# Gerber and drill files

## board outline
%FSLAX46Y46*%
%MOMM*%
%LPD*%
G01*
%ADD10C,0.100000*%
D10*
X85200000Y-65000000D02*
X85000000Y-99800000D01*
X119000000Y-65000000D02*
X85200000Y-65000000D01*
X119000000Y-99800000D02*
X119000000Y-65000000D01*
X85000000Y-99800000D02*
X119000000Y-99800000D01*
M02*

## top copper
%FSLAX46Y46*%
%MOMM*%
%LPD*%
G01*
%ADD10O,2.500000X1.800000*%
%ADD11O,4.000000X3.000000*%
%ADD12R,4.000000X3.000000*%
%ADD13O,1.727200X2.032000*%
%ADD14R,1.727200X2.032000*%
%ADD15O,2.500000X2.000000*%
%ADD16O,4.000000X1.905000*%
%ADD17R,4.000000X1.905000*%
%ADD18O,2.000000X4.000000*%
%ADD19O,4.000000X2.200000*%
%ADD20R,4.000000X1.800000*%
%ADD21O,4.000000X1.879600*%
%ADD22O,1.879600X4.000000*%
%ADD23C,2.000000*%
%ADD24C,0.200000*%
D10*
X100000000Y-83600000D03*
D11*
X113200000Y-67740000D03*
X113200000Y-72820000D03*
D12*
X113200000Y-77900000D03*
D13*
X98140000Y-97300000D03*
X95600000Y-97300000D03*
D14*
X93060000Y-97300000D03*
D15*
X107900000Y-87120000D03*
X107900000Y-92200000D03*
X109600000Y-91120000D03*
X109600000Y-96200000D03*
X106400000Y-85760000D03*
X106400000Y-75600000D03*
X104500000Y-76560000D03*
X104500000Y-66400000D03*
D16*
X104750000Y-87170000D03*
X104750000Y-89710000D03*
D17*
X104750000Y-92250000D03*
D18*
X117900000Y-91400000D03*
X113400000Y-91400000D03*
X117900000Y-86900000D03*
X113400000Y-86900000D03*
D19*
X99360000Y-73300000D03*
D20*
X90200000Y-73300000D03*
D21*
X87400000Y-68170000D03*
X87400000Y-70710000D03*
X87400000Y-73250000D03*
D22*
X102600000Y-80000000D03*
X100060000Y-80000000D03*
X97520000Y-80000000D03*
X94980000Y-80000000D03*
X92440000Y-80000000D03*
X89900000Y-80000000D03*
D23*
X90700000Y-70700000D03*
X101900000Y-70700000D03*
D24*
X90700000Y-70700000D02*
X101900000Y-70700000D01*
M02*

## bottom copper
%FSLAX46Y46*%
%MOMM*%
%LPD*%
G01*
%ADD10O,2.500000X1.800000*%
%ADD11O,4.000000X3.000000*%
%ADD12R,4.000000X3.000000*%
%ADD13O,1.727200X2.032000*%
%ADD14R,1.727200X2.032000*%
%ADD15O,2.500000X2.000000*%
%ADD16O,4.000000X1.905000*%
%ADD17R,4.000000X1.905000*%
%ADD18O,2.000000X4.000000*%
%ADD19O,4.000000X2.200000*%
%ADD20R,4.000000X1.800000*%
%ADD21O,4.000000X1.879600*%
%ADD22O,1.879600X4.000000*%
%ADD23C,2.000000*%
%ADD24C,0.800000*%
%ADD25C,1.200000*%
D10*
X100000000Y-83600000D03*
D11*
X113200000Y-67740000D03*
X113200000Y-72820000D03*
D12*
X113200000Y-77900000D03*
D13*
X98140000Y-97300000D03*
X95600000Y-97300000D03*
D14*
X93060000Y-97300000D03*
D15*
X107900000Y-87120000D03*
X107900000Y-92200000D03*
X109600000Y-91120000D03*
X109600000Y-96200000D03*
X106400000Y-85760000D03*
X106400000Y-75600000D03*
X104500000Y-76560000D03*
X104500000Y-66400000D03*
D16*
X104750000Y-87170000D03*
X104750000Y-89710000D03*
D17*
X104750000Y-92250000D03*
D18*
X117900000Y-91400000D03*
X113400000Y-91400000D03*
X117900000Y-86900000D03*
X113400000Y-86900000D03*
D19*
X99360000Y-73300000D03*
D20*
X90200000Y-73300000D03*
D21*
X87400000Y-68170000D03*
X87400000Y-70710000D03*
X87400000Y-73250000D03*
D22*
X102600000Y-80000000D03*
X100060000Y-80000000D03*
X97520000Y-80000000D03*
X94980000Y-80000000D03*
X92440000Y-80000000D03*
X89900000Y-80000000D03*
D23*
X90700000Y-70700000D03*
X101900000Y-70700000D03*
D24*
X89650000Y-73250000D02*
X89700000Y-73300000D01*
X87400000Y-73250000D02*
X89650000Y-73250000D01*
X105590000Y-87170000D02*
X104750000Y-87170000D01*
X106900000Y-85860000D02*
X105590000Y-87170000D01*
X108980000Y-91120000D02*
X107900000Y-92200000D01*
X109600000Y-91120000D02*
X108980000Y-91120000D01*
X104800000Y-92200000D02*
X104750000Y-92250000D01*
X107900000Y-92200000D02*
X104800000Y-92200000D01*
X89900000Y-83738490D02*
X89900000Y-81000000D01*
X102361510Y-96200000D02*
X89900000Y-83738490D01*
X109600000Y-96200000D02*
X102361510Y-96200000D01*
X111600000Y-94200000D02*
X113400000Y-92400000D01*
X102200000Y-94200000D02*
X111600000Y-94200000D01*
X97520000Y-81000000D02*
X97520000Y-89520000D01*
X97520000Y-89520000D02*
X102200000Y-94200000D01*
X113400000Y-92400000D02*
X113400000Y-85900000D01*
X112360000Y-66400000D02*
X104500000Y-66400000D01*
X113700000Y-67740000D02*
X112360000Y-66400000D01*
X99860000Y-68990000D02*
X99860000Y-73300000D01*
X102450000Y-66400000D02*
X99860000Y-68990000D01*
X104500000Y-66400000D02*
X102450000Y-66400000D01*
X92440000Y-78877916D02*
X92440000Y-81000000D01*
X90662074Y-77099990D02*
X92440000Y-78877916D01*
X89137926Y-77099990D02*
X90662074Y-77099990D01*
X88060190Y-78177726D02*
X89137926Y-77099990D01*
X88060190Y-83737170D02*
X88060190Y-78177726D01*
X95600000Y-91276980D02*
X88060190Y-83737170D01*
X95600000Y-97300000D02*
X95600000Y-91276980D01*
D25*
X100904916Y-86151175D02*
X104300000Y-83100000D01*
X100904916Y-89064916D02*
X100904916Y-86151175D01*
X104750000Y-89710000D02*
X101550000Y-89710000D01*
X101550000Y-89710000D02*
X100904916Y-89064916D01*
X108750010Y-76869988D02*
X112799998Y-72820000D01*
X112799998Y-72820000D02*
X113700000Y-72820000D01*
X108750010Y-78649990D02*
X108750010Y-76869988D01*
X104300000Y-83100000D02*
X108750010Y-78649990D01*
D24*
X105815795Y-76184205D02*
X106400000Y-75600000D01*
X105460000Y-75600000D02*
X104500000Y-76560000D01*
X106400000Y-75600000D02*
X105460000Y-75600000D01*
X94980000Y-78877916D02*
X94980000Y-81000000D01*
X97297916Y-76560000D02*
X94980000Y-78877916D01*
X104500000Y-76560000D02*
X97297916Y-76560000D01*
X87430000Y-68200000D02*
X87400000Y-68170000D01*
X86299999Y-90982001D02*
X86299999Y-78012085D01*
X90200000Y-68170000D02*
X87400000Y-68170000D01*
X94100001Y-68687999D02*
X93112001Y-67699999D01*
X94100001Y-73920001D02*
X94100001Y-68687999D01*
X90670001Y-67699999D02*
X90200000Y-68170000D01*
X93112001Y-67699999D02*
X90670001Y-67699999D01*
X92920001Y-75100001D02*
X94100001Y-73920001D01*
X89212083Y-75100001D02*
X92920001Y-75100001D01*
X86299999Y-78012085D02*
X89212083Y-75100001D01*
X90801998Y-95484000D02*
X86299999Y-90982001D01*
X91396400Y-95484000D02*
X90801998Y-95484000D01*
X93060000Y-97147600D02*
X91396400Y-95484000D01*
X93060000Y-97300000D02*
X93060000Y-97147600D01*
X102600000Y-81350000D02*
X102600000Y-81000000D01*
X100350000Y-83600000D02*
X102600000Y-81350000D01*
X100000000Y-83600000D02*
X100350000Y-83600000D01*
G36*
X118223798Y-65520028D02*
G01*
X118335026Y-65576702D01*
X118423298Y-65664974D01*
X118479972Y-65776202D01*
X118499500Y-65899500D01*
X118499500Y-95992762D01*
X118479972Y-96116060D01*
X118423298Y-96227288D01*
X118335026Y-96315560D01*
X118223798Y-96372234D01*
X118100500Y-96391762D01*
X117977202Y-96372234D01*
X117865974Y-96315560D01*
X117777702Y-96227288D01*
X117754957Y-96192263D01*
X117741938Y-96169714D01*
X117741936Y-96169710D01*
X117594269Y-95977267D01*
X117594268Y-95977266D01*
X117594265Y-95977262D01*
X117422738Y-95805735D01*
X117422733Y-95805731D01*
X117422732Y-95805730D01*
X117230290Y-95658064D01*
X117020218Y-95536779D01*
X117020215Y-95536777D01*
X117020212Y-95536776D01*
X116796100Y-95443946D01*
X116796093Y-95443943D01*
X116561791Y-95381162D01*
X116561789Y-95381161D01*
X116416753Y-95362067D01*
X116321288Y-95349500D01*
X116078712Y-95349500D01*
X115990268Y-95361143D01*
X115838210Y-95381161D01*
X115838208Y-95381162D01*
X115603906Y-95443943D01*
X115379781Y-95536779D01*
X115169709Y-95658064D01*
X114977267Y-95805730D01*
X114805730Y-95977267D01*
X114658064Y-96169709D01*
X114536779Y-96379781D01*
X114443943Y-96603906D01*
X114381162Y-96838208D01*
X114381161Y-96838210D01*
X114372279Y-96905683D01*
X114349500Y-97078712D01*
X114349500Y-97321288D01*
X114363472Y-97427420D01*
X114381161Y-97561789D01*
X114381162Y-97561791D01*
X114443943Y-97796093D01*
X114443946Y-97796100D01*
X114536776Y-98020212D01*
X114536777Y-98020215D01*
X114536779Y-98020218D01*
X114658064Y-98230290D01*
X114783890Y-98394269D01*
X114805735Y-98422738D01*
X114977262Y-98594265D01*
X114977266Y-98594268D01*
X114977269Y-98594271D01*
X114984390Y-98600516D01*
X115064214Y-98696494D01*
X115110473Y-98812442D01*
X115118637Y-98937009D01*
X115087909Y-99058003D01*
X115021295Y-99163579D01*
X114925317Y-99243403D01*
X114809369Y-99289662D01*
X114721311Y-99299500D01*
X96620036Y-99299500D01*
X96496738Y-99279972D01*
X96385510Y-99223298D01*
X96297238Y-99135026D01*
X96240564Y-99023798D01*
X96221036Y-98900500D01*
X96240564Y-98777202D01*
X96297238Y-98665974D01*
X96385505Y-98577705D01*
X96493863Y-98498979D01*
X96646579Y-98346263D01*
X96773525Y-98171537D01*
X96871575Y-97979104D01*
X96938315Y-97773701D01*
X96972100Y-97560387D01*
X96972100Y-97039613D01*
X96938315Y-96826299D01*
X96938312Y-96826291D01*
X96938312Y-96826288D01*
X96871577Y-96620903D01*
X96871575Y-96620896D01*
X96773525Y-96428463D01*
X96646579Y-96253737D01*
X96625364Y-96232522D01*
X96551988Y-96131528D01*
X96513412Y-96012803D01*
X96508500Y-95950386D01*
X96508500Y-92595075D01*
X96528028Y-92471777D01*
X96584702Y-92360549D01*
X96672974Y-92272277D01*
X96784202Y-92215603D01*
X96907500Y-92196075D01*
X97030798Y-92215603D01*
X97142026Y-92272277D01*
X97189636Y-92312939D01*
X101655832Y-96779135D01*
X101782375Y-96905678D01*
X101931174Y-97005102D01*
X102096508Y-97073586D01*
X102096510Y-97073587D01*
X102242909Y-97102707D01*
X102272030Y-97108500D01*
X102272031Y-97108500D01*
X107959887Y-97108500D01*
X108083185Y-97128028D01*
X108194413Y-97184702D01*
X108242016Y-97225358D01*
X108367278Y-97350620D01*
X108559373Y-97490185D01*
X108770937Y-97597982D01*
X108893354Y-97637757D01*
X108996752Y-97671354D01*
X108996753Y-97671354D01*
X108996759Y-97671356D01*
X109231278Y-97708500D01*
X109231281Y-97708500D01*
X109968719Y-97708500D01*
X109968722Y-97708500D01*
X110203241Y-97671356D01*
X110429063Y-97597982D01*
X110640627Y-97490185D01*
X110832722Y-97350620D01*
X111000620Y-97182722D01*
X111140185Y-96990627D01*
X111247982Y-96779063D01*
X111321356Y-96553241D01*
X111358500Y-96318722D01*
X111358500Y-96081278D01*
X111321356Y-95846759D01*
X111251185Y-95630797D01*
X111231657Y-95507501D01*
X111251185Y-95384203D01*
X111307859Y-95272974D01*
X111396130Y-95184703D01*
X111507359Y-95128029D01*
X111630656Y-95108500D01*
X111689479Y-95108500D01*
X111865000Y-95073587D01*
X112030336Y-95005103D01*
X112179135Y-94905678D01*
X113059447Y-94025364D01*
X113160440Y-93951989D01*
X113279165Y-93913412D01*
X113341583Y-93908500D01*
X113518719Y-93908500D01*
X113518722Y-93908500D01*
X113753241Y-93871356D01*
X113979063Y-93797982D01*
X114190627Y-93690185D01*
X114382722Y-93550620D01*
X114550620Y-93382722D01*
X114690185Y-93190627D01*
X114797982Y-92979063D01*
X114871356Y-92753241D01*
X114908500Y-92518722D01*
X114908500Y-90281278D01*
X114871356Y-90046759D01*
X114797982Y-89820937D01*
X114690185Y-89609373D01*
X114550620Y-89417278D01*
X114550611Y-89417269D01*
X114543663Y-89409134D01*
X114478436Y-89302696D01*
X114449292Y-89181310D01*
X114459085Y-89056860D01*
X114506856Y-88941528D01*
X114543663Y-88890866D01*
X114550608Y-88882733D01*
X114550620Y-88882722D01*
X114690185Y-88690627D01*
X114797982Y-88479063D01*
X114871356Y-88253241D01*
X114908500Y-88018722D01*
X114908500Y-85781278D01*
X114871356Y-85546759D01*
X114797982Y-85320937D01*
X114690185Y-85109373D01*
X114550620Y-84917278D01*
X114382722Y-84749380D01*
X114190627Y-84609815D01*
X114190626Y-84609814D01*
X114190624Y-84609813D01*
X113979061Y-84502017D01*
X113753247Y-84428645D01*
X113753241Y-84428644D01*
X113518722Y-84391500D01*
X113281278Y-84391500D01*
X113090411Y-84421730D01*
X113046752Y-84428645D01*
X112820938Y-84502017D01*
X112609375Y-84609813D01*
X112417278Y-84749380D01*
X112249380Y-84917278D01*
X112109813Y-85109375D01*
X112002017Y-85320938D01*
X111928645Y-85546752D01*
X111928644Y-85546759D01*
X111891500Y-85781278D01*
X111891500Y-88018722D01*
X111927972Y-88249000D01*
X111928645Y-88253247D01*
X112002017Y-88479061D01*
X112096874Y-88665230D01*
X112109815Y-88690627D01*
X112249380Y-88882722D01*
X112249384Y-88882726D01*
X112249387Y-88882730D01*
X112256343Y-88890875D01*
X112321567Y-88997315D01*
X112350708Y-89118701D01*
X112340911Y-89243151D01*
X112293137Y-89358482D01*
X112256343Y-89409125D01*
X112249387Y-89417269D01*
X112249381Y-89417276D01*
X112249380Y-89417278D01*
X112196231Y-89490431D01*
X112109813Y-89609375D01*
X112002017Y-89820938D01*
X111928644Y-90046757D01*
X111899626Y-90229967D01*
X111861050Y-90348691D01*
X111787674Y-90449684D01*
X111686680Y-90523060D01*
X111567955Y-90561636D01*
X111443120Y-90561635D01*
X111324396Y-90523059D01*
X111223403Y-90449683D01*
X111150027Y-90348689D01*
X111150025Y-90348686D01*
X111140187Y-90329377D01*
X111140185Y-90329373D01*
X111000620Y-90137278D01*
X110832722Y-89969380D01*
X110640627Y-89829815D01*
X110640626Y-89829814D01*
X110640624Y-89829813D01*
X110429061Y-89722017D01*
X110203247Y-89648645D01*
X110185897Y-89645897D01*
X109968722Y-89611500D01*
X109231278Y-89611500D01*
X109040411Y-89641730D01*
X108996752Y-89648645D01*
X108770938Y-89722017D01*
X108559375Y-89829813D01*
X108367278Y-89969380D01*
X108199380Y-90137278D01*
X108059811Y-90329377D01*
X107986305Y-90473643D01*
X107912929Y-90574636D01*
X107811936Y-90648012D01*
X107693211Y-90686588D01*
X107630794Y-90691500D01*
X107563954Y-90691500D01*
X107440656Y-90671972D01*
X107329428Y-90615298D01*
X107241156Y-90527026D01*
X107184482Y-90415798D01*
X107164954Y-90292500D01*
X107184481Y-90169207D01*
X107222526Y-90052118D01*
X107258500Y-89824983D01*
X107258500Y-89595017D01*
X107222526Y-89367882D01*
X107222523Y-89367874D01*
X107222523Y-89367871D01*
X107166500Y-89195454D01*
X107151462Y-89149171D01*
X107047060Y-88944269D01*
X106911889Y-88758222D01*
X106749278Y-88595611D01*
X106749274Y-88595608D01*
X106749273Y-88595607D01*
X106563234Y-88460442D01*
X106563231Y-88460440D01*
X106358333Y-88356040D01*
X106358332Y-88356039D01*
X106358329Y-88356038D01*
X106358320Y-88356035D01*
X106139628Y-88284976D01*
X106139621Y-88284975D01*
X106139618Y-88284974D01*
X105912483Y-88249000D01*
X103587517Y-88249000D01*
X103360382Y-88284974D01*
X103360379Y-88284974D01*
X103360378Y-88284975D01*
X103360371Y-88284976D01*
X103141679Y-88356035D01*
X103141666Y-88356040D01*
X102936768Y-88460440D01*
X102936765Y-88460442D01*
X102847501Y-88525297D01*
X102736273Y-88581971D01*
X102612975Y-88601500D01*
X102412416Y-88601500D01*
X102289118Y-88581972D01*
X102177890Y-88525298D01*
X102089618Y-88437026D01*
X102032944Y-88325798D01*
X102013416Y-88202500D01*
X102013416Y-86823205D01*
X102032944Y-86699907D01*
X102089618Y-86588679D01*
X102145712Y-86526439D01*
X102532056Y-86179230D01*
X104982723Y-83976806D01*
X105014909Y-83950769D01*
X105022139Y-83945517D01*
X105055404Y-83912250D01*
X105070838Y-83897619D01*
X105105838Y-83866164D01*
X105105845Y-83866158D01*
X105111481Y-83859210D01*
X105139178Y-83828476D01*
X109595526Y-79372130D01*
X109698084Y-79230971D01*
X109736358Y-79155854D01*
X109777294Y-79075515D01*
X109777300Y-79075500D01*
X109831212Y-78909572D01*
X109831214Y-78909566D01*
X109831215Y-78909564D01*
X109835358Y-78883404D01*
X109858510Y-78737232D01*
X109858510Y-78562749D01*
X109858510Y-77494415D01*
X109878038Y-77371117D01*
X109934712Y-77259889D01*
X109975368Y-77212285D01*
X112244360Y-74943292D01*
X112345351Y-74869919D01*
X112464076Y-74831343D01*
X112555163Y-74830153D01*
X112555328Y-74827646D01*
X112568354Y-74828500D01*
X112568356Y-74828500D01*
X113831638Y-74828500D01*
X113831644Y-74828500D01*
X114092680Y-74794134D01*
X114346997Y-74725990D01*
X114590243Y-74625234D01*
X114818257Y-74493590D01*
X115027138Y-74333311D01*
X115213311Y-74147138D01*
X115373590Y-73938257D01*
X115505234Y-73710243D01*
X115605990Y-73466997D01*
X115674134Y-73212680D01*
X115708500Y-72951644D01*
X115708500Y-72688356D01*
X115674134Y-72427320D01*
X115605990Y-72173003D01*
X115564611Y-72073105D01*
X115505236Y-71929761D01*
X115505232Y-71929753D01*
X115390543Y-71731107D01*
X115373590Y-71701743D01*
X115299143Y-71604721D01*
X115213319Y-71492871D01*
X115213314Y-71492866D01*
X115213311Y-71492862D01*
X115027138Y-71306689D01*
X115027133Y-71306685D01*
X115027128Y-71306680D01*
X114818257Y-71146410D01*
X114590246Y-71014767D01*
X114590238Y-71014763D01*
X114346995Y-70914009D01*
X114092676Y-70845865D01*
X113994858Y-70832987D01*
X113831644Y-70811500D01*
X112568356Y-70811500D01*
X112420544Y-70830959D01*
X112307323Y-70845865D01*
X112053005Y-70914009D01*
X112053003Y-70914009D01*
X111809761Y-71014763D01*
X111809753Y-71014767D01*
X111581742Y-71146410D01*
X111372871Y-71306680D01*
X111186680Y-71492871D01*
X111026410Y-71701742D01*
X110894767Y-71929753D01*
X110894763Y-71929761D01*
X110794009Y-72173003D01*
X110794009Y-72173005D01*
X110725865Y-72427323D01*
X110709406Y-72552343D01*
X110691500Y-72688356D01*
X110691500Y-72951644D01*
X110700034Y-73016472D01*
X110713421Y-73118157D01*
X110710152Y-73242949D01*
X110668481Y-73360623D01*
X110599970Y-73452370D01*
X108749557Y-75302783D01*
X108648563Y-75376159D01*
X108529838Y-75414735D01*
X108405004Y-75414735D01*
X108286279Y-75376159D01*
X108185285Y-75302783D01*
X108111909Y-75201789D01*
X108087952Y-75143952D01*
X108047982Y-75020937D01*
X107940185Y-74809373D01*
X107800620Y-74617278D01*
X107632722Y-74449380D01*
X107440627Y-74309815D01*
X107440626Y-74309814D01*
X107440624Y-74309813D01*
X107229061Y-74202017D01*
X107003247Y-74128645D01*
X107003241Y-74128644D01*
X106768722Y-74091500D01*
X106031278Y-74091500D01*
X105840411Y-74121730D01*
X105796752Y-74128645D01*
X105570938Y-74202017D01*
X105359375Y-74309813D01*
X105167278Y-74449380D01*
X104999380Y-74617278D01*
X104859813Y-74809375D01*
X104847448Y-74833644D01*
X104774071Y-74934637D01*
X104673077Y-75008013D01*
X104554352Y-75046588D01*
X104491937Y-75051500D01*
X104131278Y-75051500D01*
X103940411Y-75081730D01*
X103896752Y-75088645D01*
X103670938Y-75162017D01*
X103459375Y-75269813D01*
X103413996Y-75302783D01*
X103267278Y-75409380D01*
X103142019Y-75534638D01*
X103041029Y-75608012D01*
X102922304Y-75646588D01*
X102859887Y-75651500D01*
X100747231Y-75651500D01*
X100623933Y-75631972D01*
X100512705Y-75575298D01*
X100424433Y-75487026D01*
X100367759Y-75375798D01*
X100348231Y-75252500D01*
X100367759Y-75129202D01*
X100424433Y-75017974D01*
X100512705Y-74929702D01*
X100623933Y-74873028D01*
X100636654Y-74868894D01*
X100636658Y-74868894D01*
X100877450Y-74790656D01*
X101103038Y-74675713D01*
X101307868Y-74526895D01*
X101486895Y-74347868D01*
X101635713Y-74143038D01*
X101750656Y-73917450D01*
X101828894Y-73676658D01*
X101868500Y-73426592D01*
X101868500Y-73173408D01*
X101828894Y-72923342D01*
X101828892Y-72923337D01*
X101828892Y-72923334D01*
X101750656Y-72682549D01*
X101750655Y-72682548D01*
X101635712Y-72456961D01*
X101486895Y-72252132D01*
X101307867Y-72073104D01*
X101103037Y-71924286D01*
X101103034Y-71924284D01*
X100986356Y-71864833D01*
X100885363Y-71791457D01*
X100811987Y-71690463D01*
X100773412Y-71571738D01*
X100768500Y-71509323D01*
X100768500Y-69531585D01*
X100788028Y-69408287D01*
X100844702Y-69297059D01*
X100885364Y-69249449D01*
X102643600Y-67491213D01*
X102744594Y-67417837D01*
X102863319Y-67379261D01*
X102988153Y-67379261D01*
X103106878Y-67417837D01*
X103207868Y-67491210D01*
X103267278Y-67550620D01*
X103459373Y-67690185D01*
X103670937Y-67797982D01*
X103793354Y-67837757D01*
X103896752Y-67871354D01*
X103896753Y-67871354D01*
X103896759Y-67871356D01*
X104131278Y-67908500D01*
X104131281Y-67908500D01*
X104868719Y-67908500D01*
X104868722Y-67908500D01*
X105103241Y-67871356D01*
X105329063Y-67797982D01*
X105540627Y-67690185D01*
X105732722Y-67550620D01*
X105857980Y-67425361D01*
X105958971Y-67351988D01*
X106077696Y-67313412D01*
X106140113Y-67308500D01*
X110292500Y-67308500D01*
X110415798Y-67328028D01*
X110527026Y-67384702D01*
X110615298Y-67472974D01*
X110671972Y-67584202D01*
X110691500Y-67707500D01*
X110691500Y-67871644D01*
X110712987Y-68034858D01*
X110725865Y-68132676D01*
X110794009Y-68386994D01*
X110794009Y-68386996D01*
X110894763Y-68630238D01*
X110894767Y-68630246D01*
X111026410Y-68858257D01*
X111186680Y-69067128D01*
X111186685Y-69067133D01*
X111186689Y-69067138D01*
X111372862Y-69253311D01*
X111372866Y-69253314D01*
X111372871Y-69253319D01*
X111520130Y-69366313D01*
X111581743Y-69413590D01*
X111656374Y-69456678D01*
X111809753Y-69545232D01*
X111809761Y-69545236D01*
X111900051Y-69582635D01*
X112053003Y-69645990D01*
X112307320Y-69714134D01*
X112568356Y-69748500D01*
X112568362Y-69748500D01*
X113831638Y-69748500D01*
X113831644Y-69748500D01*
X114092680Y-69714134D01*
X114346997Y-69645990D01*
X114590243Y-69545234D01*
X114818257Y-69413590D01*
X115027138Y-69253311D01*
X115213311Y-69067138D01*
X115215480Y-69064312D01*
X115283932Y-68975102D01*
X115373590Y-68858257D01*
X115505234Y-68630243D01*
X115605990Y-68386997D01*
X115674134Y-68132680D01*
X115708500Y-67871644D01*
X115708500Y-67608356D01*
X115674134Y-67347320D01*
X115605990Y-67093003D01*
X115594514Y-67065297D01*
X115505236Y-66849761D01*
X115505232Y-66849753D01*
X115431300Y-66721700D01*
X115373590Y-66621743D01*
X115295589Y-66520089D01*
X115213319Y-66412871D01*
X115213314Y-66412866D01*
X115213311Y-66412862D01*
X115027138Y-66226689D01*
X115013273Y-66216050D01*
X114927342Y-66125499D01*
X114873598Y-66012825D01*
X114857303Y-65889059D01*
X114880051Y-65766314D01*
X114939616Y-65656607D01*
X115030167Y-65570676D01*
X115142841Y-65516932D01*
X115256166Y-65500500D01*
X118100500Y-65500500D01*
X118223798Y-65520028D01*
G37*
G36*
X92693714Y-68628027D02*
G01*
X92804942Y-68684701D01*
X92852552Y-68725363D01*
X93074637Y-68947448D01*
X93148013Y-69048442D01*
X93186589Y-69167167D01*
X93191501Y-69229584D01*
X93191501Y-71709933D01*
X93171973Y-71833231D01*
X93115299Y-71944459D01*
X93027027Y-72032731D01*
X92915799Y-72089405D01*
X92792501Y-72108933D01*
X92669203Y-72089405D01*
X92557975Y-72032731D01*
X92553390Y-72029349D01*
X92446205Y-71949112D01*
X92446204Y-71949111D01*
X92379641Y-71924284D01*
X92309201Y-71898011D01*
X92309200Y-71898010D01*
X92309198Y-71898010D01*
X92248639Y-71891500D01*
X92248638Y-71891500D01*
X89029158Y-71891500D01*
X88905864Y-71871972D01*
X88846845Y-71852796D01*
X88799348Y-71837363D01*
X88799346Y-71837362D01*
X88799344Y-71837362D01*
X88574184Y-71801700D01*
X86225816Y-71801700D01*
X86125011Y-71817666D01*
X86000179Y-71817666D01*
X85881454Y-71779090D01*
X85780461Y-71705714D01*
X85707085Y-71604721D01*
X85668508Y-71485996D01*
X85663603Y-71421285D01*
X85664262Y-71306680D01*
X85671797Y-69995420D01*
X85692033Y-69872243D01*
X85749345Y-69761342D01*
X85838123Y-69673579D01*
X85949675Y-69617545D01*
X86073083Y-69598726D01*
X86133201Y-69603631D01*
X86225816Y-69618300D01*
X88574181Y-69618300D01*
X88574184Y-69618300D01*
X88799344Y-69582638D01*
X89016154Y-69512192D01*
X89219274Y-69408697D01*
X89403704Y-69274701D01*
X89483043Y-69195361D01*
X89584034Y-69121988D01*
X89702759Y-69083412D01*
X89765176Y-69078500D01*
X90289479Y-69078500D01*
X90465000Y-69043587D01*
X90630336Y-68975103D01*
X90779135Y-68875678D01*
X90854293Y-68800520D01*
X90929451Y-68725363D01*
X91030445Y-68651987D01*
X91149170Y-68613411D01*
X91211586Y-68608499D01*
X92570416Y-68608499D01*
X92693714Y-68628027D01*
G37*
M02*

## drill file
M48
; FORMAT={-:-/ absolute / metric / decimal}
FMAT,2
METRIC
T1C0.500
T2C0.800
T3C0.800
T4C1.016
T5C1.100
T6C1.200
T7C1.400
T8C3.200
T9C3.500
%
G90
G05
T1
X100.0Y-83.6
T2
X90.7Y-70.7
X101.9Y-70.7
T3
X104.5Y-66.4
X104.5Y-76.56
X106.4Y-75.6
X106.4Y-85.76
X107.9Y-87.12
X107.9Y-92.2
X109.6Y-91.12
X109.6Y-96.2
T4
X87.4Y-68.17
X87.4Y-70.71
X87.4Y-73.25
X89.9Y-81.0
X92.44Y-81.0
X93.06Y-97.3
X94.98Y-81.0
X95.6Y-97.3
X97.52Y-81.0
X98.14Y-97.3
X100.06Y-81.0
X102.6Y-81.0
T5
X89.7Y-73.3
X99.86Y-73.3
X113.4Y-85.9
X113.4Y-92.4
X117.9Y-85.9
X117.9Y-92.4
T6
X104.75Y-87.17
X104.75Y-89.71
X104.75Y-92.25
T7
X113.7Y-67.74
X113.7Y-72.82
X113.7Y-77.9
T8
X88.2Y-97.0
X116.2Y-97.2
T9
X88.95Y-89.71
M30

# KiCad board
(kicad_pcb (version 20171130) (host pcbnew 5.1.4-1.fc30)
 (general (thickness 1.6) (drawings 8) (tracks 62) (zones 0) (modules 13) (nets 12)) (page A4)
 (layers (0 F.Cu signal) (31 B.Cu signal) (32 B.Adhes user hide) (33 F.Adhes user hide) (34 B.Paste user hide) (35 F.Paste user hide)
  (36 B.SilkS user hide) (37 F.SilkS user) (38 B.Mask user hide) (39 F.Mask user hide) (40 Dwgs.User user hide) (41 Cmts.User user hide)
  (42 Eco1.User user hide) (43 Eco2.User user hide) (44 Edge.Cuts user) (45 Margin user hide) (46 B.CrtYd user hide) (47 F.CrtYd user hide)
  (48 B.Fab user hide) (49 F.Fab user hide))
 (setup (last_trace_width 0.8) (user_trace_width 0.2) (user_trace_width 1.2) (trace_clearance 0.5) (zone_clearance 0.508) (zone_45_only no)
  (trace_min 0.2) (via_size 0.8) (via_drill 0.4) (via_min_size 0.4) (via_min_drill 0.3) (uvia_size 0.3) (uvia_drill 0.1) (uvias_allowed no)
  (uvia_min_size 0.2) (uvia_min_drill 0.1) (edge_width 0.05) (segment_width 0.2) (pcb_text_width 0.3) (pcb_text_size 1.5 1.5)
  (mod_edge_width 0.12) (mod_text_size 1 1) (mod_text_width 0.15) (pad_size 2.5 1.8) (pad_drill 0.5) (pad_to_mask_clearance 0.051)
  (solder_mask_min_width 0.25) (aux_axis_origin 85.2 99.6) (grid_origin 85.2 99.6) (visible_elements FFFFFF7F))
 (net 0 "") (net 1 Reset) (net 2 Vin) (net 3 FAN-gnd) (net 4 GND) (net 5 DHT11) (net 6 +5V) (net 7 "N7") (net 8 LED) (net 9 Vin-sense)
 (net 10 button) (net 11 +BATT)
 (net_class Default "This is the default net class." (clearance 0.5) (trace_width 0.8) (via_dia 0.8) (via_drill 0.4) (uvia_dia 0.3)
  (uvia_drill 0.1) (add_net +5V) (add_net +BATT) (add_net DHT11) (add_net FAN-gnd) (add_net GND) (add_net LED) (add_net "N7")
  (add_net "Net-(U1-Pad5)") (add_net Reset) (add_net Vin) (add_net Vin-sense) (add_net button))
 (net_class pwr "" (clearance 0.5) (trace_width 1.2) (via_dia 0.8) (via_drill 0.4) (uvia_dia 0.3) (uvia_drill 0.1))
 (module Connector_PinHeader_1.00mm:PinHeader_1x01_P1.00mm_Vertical (layer F.Cu) (at 100 83.6)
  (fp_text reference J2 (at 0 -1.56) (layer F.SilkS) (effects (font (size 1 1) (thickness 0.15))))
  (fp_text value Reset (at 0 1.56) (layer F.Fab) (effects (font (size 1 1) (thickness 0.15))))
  (pad 1 thru_hole oval (at 0 0) (size 2.5 1.8) (drill 0.5) (layers *.Cu *.Mask) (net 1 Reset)))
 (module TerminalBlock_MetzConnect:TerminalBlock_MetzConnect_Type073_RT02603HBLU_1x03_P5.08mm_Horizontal (layer F.Cu) (at 113.7 77.9 90)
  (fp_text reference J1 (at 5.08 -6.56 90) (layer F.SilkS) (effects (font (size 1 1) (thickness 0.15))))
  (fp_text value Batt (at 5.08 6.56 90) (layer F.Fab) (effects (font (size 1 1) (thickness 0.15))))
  (pad 3 thru_hole oval (at 10.16 0 90) (size 3 4) (drill 1.4 (offset 0 -0.5)) (layers *.Cu *.Mask) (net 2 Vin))
  (pad 2 thru_hole oval (at 5.08 0 90) (size 3 4) (drill 1.4 (offset 0 -0.5)) (layers *.Cu *.Mask) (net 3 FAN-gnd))
  (pad 1 thru_hole rect (at 0 0 90) (size 3 4) (drill 1.4 (offset 0 -0.5)) (layers *.Cu *.Mask) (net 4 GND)))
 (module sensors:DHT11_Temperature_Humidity (layer F.Cu) (at 95.6 97.3)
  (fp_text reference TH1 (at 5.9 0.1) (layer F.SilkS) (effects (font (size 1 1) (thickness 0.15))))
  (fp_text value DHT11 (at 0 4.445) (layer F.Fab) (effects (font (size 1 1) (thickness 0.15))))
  (pad 3 thru_hole oval (at 2.54 0 90) (size 2.032 1.7272) (drill 1.016) (layers *.Cu *.Mask F.SilkS) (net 4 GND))
  (pad 2 thru_hole oval (at 0 0 90) (size 2.032 1.7272) (drill 1.016) (layers *.Cu *.Mask F.SilkS) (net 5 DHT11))
  (pad 1 thru_hole rect (at -2.54 0 90) (size 2.032 1.7272) (drill 1.016) (layers *.Cu *.Mask F.SilkS) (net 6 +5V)))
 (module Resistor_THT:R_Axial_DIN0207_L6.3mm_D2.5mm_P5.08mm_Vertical (layer F.Cu) (at 107.9 92.2 90)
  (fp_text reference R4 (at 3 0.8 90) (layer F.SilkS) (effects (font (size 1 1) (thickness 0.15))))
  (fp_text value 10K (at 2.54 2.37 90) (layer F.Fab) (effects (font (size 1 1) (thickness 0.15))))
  (pad 2 thru_hole oval (at 5.08 0 90) (size 2 2.5) (drill 0.8) (layers *.Cu *.Mask) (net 4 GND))
  (pad 1 thru_hole oval (at 0 0 90) (size 2 2.5) (drill 0.8) (layers *.Cu *.Mask) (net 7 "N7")))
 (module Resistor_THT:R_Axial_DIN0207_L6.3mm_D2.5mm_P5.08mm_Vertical (layer F.Cu) (at 109.6 96.2 90)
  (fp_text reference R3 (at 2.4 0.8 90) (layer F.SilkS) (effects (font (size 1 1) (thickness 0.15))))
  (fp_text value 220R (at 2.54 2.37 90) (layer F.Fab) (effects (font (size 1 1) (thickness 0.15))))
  (pad 2 thru_hole oval (at 5.08 0 90) (size 2 2.5) (drill 0.8) (layers *.Cu *.Mask) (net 7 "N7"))
  (pad 1 thru_hole oval (at 0 0 90) (size 2 2.5) (drill 0.8) (layers *.Cu *.Mask) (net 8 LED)))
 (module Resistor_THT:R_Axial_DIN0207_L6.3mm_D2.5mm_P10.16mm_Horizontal (layer F.Cu) (at 106.4 75.6 270)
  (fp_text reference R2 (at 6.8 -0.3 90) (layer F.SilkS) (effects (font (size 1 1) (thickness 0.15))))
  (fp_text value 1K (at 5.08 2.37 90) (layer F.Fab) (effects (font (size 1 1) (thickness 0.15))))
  (pad 2 thru_hole oval (at 10.16 0 270) (size 2 2.5) (drill 0.8) (layers *.Cu *.Mask) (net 4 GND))
  (pad 1 thru_hole oval (at 0 0 270) (size 2 2.5) (drill 0.8) (layers *.Cu *.Mask) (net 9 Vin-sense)))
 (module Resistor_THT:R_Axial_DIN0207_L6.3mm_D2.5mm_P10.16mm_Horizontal (layer F.Cu) (at 104.5 66.4 270)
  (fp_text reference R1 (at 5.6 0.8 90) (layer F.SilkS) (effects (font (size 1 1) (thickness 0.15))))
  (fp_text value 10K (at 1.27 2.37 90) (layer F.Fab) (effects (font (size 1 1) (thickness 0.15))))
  (pad 2 thru_hole oval (at 10.16 0 270) (size 2 2.5) (drill 0.8) (layers *.Cu *.Mask) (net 9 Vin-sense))
  (pad 1 thru_hole oval (at 0 0 270) (size 2 2.5) (drill 0.8) (layers *.Cu *.Mask) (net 2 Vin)))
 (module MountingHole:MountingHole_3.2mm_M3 (layer F.Cu) (at 116.2 97.2)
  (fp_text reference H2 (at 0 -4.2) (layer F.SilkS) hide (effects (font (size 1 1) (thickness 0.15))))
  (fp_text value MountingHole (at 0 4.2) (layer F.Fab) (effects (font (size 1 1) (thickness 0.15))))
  (pad 1 np_thru_hole circle (at 0 0) (size 3.2 3.2) (drill 3.2) (layers *.Cu *.Mask)))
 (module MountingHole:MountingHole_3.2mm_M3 (layer F.Cu) (at 88.2 97)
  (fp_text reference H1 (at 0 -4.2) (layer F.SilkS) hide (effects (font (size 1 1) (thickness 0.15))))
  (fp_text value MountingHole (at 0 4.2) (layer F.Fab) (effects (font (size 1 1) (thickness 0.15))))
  (pad 1 np_thru_hole circle (at 0 0) (size 3.2 3.2) (drill 3.2) (layers *.Cu *.Mask)))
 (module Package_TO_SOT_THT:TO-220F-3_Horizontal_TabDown (layer F.Cu) (at 104.75 92.25 90)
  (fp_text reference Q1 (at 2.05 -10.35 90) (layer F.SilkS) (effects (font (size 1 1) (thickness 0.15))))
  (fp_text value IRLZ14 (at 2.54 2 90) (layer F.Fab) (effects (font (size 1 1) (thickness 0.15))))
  (pad 3 thru_hole oval (at 5.08 0 90) (size 1.905 4) (drill 1.2) (layers *.Cu *.Mask) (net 4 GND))
  (pad 2 thru_hole oval (at 2.54 0 90) (size 1.905 4) (drill 1.2) (layers *.Cu *.Mask) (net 3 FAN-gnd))
  (pad 1 thru_hole rect (at 0 0 90) (size 1.905 4) (drill 1.2) (layers *.Cu *.Mask) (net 7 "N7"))
  (pad "" np_thru_hole oval (at 2.54 -15.8 90) (size 3.5 3.5) (drill 3.5) (layers *.Cu *.Mask)))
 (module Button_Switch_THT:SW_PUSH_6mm (layer F.Cu) (at 117.9 85.9 270)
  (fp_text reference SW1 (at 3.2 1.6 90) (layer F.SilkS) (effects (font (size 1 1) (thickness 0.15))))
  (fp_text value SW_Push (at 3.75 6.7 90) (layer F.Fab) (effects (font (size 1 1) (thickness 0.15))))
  (pad 1 thru_hole oval (at 6.5 0 270) (size 4 2) (drill 1.1 (offset -1 0)) (layers *.Cu *.Mask) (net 4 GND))
  (pad 2 thru_hole oval (at 6.5 4.5) (size 2 4) (drill 1.1 (offset 0 -1)) (layers *.Cu *.Mask) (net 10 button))
  (pad 1 thru_hole oval (at 0 0) (size 2 4) (drill 1.1 (offset 0 1)) (layers *.Cu *.Mask) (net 4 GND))
  (pad 2 thru_hole oval (at 0 4.5) (size 2 4) (drill 1.1 (offset 0 1)) (layers *.Cu *.Mask) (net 10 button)))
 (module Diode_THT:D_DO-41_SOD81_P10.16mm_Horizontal (layer F.Cu) (at 89.7 73.3)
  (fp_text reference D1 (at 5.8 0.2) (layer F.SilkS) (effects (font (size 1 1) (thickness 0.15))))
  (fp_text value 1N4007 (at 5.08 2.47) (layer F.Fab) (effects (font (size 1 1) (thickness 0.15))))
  (pad 2 thru_hole oval (at 10.16 0) (size 4 2.2) (drill 1.1 (offset -0.5 0)) (layers *.Cu *.Mask) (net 2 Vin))
  (pad 1 thru_hole rect (at 0 0) (size 4 1.8) (drill 1.1 (offset 0.5 0)) (layers *.Cu *.Mask) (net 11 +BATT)))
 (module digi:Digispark (layer F.Cu) (at 96.25 81)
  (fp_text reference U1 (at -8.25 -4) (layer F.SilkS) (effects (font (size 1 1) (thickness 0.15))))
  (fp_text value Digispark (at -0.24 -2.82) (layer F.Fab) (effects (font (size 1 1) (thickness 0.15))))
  (pad 9 thru_hole oval (at -8.85 -12.83) (size 4 1.8796) (drill 1.016) (layers *.Cu *.Mask) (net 6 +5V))
  (pad 8 thru_hole oval (at -8.85 -10.29) (size 4 1.8796) (drill 1.016) (layers *.Cu *.Mask) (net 4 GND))
  (pad 7 thru_hole oval (at -8.85 -7.75) (size 4 1.8796) (drill 1.016) (layers *.Cu *.Mask) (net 11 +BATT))
  (pad 6 thru_hole oval (at 6.35 0) (size 1.8796 4) (drill 1.016 (offset 0 -1)) (layers *.Cu *.Mask) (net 1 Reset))
  (pad 5 thru_hole oval (at 3.81 0) (size 1.8796 4) (drill 1.016 (offset 0 -1)) (layers *.Cu *.Mask))
  (pad 4 thru_hole oval (at 1.27 0) (size 1.8796 4) (drill 1.016 (offset 0 -1)) (layers *.Cu *.Mask) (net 10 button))
  (pad 3 thru_hole oval (at -1.27 0) (size 1.8796 4) (drill 1.016 (offset 0 -1)) (layers *.Cu *.Mask) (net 9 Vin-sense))
  (pad 2 thru_hole oval (at -3.81 0) (size 1.8796 4) (drill 1.016 (offset 0 -1)) (layers *.Cu *.Mask) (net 5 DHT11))
  (pad 1 thru_hole oval (at -6.35 0) (size 1.8796 4) (drill 1.016 (offset 0 -1)) (layers *.Cu *.Mask) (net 8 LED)))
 (gr_line (start 85.2 65) (end 85 99.8) (layer Edge.Cuts) (width 0.1))
 (gr_line (start 119 65) (end 85.2 65) (layer Edge.Cuts) (width 0.1))
 (gr_line (start 119 99.8) (end 119 65) (layer Edge.Cuts) (width 0.1))
 (gr_line (start 85 99.8) (end 119 99.8) (layer Edge.Cuts) (width 0.1))
 (segment (start 89.65 73.25) (end 89.7 73.3) (width 0.8) (layer B.Cu) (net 11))
 (segment (start 87.4 73.25) (end 89.65 73.25) (width 0.8) (layer B.Cu) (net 11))
 (segment (start 105.59 87.17) (end 104.75 87.17) (width 0.8) (layer B.Cu) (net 4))
 (segment (start 106.9 85.86) (end 105.59 87.17) (width 0.8) (layer B.Cu) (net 4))
 (via (at 90.7 70.7) (size 2) (drill 0.8) (layers F.Cu B.Cu) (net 4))
 (via (at 101.9 70.7) (size 2) (drill 0.8) (layers F.Cu B.Cu) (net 4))
 (segment (start 90.7 70.7) (end 101.9 70.7) (width 0.2) (layer F.Cu) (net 4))
 (segment (start 108.98 91.12) (end 107.9 92.2) (width 0.8) (layer B.Cu) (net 7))
 (segment (start 109.6 91.12) (end 108.98 91.12) (width 0.8) (layer B.Cu) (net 7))
 (segment (start 104.8 92.2) (end 104.75 92.25) (width 0.8) (layer B.Cu) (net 7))
 (segment (start 107.9 92.2) (end 104.8 92.2) (width 0.8) (layer B.Cu) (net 7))
 (segment (start 89.9 83.73849) (end 89.9 81) (width 0.8) (layer B.Cu) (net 8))
 (segment (start 102.36151 96.2) (end 89.9 83.73849) (width 0.8) (layer B.Cu) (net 8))
 (segment (start 109.6 96.2) (end 102.36151 96.2) (width 0.8) (layer B.Cu) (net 8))
 (segment (start 111.6 94.2) (end 113.4 92.4) (width 0.8) (layer B.Cu) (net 10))
 (segment (start 102.2 94.2) (end 111.6 94.2) (width 0.8) (layer B.Cu) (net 10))
 (segment (start 97.52 81) (end 97.52 89.52) (width 0.8) (layer B.Cu) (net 10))
 (segment (start 97.52 89.52) (end 102.2 94.2) (width 0.8) (layer B.Cu) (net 10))
 (segment (start 113.4 92.4) (end 113.4 85.9) (width 0.8) (layer B.Cu) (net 10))
 (segment (start 112.36 66.4) (end 104.5 66.4) (width 0.8) (layer B.Cu) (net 2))
 (segment (start 113.7 67.74) (end 112.36 66.4) (width 0.8) (layer B.Cu) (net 2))
 (segment (start 99.86 68.99) (end 99.86 73.3) (width 0.8) (layer B.Cu) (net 2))
 (segment (start 102.45 66.4) (end 99.86 68.99) (width 0.8) (layer B.Cu) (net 2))
 (segment (start 104.5 66.4) (end 102.45 66.4) (width 0.8) (layer B.Cu) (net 2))
 (segment (start 92.44 78.877916) (end 92.44 81) (width 0.8) (layer B.Cu) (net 5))
 (segment (start 90.662074 77.09999) (end 92.44 78.877916) (width 0.8) (layer B.Cu) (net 5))
 (segment (start 89.137926 77.09999) (end 90.662074 77.09999) (width 0.8) (layer B.Cu) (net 5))
 (segment (start 88.06019 78.177726) (end 89.137926 77.09999) (width 0.8) (layer B.Cu) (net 5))
 (segment (start 88.06019 83.73717) (end 88.06019 78.177726) (width 0.8) (layer B.Cu) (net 5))
 (segment (start 95.6 91.27698) (end 88.06019 83.73717) (width 0.8) (layer B.Cu) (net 5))
 (segment (start 95.6 97.3) (end 95.6 91.27698) (width 0.8) (layer B.Cu) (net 5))
 (segment (start 100.904916 86.151175) (end 104.3 83.1) (width 1.2) (layer B.Cu) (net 3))
 (segment (start 100.904916 89.064916) (end 100.904916 86.151175) (width 1.2) (layer B.Cu) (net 3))
 (segment (start 104.75 89.71) (end 101.55 89.71) (width 1.2) (layer B.Cu) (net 3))
 (segment (start 101.55 89.71) (end 100.904916 89.064916) (width 1.2) (layer B.Cu) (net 3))
 (segment (start 108.75001 76.869988) (end 112.799998 72.82) (width 1.2) (layer B.Cu) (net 3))
 (segment (start 112.799998 72.82) (end 113.7 72.82) (width 1.2) (layer B.Cu) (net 3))
 (segment (start 108.75001 78.64999) (end 108.75001 76.869988) (width 1.2) (layer B.Cu) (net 3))
 (segment (start 104.3 83.1) (end 108.75001 78.64999) (width 1.2) (layer B.Cu) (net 3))
 (segment (start 105.815795 76.184205) (end 106.4 75.6) (width 0.8) (layer B.Cu) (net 9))
 (segment (start 105.46 75.6) (end 104.5 76.56) (width 0.8) (layer B.Cu) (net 9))
 (segment (start 106.4 75.6) (end 105.46 75.6) (width 0.8) (layer B.Cu) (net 9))
 (segment (start 94.98 78.877916) (end 94.98 81) (width 0.8) (layer B.Cu) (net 9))
 (segment (start 97.297916 76.56) (end 94.98 78.877916) (width 0.8) (layer B.Cu) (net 9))
 (segment (start 104.5 76.56) (end 97.297916 76.56) (width 0.8) (layer B.Cu) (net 9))
 (segment (start 87.43 68.2) (end 87.4 68.17) (width 0.8) (layer B.Cu) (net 6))
 (segment (start 86.299999 90.982001) (end 86.299999 78.012085) (width 0.8) (layer B.Cu) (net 6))
 (segment (start 90.2 68.17) (end 87.4 68.17) (width 0.8) (layer B.Cu) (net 6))
 (segment (start 94.100001 68.687999) (end 93.112001 67.699999) (width 0.8) (layer B.Cu) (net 6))
 (segment (start 94.100001 73.920001) (end 94.100001 68.687999) (width 0.8) (layer B.Cu) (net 6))
 (segment (start 90.670001 67.699999) (end 90.2 68.17) (width 0.8) (layer B.Cu) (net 6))
 (segment (start 93.112001 67.699999) (end 90.670001 67.699999) (width 0.8) (layer B.Cu) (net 6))
 (segment (start 92.920001 75.100001) (end 94.100001 73.920001) (width 0.8) (layer B.Cu) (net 6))
 (segment (start 89.212083 75.100001) (end 92.920001 75.100001) (width 0.8) (layer B.Cu) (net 6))
 (segment (start 86.299999 78.012085) (end 89.212083 75.100001) (width 0.8) (layer B.Cu) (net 6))
 (segment (start 90.801998 95.484) (end 86.299999 90.982001) (width 0.8) (layer B.Cu) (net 6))
 (segment (start 91.3964 95.484) (end 90.801998 95.484) (width 0.8) (layer B.Cu) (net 6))
 (segment (start 93.06 97.1476) (end 91.3964 95.484) (width 0.8) (layer B.Cu) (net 6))
 (segment (start 93.06 97.3) (end 93.06 97.1476) (width 0.8) (layer B.Cu) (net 6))
 (segment (start 102.6 81.35) (end 102.6 81) (width 0.8) (layer B.Cu) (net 1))
 (segment (start 100.35 83.6) (end 102.6 81.35) (width 0.8) (layer B.Cu) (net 1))
 (segment (start 100 83.6) (end 100.35 83.6) (width 0.8) (layer B.Cu) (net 1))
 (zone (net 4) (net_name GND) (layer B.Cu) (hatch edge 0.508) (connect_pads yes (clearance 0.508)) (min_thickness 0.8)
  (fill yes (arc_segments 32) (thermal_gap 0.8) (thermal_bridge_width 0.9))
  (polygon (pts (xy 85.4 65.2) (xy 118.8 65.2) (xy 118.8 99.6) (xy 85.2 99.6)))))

